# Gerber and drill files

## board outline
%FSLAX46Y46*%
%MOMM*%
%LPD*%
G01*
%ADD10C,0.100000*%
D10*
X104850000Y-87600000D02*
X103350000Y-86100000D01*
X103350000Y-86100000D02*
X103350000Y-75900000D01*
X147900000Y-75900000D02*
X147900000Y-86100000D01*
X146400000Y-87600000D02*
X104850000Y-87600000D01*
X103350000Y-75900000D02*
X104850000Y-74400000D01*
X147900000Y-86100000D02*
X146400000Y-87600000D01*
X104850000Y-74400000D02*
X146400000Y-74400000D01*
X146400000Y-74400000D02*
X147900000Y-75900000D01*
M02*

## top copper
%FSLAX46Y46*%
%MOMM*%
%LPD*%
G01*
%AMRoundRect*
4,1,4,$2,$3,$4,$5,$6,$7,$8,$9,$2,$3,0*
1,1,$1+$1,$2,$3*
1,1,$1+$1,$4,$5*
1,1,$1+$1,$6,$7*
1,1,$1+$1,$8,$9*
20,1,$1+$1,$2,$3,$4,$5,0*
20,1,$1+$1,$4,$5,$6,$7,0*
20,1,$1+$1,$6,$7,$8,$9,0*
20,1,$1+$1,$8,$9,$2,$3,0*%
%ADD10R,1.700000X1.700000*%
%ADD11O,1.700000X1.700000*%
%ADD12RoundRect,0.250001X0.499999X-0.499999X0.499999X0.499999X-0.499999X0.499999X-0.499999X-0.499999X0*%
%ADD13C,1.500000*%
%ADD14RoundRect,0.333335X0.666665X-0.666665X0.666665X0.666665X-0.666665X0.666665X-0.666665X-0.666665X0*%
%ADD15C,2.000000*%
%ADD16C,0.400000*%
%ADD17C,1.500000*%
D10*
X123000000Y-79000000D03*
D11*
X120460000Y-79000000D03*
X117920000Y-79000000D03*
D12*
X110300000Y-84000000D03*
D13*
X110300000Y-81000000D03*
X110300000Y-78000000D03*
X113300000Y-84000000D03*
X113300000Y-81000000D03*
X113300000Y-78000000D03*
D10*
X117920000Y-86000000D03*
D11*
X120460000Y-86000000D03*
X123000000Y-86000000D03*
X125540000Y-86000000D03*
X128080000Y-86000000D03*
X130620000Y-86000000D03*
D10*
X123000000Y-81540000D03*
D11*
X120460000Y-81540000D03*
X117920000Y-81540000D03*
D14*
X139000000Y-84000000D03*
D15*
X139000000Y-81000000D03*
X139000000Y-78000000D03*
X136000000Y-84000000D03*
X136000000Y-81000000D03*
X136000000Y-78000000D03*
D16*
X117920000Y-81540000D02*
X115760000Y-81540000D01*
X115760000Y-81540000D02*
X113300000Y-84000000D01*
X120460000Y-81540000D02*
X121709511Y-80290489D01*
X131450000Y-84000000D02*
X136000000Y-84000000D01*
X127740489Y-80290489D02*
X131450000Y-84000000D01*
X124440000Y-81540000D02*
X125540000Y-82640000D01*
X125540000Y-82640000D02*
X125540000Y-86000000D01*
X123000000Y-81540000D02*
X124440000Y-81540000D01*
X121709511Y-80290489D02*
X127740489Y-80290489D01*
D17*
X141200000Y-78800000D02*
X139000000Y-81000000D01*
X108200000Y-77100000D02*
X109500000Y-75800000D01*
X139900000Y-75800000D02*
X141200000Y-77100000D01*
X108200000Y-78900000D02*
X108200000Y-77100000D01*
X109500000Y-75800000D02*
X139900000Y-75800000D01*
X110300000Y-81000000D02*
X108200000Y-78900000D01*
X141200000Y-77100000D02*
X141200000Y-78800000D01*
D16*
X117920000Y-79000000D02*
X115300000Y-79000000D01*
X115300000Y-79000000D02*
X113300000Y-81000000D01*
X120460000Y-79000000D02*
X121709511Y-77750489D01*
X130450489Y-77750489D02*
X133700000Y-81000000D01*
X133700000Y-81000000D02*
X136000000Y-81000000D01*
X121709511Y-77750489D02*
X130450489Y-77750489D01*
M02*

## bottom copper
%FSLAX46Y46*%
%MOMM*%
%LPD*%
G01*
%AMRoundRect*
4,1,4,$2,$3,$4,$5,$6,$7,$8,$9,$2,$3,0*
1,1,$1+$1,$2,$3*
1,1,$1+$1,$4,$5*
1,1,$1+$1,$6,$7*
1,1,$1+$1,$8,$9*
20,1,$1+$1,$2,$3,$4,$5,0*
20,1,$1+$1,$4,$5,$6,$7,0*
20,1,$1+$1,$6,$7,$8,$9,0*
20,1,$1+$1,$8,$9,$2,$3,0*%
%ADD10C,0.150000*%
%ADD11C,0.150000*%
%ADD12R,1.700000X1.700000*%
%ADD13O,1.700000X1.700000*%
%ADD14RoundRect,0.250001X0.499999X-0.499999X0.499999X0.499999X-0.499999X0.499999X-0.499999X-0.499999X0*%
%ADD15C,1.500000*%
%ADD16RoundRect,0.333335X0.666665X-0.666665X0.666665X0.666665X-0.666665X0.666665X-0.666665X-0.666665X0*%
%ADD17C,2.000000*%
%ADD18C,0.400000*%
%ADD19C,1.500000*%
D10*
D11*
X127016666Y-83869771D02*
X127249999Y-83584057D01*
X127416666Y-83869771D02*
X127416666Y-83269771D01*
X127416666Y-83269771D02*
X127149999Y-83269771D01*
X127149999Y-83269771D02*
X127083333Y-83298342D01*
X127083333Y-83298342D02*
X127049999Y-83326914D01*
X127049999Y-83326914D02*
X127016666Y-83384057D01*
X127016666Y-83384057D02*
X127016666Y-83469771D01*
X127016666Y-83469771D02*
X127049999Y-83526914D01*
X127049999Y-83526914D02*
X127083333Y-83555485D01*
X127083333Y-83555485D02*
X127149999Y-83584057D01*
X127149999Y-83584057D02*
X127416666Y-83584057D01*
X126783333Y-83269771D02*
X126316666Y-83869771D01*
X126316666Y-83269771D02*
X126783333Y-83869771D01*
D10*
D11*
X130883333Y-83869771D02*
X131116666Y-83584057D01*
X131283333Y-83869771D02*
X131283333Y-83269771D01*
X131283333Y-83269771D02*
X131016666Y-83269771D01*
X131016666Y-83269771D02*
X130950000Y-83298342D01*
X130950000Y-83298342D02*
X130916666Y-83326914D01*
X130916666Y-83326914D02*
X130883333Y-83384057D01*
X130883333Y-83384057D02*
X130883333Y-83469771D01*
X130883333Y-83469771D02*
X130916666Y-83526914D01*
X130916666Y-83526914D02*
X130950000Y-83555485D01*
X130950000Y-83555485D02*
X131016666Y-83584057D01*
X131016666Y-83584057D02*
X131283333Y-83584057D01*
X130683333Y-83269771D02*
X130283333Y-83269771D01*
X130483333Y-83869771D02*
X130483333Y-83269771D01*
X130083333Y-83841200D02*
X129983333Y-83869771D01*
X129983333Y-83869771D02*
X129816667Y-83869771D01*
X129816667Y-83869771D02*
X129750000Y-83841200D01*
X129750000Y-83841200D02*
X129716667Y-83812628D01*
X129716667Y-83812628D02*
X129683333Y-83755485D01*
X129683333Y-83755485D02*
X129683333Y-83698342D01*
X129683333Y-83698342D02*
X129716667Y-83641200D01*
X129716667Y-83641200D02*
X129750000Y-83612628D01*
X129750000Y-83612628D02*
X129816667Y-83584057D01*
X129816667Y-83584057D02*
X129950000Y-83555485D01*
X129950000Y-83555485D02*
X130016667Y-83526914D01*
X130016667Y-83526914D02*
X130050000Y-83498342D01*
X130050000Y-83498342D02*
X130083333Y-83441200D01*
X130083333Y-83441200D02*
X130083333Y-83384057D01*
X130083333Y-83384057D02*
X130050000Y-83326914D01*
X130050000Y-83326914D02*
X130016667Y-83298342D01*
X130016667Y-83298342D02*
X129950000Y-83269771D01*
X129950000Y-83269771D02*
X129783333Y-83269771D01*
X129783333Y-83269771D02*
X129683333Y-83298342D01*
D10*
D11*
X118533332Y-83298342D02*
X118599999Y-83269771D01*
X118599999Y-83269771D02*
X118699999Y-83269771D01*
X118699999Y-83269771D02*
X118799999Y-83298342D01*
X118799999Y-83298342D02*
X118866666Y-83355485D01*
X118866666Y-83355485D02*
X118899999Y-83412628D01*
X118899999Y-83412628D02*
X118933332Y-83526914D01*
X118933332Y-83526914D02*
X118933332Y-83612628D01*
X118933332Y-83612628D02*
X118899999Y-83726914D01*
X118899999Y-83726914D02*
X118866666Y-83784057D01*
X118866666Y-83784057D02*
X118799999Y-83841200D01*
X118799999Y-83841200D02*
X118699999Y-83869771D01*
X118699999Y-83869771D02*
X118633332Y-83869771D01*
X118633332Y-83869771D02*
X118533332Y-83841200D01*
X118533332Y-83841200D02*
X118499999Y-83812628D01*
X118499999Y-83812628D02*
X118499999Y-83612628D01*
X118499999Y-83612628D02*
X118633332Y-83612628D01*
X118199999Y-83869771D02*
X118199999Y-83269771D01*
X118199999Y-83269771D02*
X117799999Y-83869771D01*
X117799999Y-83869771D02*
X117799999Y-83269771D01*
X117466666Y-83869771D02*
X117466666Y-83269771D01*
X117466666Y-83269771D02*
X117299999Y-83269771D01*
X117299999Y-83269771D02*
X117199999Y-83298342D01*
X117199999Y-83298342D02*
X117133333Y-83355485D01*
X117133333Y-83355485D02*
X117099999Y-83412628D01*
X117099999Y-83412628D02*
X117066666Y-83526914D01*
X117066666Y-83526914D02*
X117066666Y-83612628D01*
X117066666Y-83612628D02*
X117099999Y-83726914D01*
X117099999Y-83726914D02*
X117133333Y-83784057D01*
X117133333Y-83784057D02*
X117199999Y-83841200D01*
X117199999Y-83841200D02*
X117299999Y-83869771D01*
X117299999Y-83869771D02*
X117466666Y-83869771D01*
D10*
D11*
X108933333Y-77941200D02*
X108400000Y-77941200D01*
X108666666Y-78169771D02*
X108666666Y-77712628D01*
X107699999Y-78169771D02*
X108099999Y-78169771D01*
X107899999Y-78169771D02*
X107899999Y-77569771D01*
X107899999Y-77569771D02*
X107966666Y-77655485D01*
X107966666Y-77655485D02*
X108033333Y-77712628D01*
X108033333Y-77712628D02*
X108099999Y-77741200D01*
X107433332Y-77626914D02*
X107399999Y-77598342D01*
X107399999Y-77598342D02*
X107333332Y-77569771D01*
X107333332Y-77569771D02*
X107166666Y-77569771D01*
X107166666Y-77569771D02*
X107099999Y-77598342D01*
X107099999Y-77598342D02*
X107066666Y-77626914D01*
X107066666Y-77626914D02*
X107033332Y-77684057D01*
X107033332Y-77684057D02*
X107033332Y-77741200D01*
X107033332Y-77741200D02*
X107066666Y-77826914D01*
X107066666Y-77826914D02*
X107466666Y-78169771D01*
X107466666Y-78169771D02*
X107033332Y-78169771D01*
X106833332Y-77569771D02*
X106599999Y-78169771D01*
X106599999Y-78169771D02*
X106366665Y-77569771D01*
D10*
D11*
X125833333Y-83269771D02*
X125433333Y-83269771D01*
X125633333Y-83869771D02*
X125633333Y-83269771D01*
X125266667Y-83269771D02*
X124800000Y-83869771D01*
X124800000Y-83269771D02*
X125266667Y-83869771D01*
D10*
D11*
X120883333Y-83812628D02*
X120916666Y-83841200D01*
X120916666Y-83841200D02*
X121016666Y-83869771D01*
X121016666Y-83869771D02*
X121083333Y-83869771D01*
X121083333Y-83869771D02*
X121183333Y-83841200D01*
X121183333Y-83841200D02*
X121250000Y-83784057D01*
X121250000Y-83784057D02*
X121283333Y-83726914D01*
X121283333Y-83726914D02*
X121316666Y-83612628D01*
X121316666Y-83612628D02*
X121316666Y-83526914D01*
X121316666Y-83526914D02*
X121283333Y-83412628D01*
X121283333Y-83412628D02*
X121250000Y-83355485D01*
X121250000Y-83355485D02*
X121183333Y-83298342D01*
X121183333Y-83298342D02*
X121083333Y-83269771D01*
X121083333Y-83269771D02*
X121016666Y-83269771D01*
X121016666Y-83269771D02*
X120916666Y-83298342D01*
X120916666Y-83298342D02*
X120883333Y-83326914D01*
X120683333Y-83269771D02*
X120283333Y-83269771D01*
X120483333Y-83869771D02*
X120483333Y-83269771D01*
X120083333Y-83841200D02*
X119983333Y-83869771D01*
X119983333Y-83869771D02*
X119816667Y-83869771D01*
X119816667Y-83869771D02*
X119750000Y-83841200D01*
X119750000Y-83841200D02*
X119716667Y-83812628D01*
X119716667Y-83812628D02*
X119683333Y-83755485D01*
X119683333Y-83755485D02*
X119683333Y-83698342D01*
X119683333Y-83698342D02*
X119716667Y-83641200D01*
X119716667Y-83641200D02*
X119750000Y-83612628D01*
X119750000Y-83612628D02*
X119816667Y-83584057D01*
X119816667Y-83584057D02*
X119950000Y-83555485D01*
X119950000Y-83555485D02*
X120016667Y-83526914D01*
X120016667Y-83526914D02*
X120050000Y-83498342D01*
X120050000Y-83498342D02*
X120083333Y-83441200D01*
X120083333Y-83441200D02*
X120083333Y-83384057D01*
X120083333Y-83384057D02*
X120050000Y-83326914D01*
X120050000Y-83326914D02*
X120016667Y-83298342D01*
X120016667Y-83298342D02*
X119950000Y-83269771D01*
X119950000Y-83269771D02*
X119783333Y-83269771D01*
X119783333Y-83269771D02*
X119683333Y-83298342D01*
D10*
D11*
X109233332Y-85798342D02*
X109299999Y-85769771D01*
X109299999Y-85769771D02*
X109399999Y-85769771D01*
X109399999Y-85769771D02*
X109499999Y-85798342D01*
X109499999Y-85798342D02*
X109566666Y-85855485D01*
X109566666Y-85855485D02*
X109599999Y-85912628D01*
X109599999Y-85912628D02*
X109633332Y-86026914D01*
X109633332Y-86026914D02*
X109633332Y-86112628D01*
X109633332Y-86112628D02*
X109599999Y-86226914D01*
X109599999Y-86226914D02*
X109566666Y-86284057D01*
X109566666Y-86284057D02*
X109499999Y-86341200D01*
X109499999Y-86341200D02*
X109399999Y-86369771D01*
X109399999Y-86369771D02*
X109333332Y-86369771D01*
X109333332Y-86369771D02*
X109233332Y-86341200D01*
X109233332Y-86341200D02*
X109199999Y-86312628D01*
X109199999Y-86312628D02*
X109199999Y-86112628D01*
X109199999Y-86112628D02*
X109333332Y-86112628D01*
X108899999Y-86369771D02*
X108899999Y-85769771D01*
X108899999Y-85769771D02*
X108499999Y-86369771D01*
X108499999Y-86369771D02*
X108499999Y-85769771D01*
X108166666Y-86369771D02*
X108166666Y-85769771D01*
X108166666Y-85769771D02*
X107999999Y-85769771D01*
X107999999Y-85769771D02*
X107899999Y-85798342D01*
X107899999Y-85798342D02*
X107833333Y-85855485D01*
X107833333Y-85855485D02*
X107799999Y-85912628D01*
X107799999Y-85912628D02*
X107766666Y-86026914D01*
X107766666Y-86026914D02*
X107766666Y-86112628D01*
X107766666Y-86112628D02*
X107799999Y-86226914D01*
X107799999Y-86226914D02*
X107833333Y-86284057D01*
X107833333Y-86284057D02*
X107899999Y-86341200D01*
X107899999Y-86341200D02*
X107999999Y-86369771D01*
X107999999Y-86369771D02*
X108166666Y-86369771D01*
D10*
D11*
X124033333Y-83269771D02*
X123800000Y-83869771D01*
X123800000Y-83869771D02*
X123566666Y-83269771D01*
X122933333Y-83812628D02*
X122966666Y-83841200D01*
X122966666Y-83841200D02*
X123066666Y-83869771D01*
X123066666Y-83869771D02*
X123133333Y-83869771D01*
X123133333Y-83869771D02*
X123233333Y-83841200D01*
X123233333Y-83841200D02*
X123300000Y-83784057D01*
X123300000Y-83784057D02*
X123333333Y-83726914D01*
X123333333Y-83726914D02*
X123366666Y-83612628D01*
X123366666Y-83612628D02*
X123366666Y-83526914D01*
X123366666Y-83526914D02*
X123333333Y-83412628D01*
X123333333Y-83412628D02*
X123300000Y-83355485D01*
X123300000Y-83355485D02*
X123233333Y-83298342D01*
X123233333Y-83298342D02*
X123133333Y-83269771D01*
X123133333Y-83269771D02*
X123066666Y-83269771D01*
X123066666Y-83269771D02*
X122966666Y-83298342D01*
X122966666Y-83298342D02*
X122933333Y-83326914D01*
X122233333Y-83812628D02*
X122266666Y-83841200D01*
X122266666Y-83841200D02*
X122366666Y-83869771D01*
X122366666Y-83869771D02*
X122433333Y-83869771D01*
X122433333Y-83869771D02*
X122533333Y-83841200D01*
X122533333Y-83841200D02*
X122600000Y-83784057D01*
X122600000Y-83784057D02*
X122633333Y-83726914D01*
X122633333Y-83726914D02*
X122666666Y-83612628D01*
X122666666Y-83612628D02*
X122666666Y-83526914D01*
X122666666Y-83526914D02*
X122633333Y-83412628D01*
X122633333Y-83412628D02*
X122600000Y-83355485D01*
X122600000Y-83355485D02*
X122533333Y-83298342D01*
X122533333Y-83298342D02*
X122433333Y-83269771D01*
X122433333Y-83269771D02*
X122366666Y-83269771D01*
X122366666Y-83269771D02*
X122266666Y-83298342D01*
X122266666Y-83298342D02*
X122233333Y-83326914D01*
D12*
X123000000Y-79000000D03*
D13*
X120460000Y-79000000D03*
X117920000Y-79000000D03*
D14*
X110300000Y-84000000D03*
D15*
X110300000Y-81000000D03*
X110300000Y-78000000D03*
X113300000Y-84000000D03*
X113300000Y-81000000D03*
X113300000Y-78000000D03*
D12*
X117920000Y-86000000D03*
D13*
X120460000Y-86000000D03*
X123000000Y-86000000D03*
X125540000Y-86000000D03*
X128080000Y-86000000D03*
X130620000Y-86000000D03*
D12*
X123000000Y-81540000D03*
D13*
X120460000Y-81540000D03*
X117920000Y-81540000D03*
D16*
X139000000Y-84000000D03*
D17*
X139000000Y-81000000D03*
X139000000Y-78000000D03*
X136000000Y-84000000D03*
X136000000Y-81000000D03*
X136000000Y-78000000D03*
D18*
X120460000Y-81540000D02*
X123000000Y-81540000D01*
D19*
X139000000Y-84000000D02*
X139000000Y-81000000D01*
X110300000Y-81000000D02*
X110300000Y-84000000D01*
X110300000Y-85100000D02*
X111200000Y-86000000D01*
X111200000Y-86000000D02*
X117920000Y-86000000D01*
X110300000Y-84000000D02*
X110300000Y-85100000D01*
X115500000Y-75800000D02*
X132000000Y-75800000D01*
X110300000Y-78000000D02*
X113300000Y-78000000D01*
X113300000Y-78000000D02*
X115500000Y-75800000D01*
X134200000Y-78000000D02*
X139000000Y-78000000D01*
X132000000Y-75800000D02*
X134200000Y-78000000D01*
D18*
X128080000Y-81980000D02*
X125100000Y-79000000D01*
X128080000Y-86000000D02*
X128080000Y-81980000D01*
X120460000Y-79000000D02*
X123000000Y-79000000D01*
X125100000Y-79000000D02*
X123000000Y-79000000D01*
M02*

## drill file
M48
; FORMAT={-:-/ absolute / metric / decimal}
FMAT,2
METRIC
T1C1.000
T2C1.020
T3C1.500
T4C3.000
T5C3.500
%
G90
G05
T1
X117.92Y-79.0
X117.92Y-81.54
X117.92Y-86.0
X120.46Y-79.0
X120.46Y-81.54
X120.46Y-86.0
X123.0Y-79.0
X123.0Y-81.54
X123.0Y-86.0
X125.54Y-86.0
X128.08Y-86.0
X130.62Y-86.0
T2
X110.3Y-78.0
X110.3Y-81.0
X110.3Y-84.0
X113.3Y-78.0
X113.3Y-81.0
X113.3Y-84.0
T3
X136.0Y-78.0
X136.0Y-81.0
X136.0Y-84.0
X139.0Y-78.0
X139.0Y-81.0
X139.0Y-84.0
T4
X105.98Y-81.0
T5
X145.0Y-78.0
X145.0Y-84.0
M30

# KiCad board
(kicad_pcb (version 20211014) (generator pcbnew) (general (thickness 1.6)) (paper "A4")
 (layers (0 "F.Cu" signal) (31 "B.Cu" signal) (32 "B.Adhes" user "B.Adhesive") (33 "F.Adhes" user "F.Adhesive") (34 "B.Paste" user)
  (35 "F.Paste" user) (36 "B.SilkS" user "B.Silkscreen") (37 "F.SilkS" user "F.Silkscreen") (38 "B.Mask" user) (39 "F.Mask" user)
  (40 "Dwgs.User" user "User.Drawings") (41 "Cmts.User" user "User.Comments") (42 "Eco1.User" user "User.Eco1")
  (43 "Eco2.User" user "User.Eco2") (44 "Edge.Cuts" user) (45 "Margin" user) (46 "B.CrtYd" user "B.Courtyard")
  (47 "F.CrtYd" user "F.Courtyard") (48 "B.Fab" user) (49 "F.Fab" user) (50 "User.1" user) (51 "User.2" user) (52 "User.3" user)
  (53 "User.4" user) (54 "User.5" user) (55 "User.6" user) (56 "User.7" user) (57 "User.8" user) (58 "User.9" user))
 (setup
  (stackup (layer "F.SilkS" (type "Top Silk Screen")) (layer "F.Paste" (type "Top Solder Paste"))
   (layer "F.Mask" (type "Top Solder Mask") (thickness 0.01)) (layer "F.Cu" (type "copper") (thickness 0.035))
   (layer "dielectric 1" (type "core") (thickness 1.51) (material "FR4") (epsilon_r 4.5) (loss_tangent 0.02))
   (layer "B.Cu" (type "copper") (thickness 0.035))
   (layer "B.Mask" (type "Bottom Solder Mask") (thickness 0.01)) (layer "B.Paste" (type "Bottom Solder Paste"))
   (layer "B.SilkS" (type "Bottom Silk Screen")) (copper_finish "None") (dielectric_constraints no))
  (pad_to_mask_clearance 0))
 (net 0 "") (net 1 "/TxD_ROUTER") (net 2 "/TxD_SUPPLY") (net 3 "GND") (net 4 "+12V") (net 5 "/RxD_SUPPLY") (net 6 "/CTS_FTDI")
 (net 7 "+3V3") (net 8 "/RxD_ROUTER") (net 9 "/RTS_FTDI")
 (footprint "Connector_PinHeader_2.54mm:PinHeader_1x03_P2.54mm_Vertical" (layer "F.Cu") (at 123 79 -90)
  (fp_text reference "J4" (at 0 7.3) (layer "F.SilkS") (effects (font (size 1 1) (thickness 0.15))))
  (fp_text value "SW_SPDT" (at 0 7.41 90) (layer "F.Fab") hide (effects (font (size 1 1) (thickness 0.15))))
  (pad "1" thru_hole rect (at 0 0 270) (size 1.7 1.7) (drill 1) (layers *.Cu *.Mask) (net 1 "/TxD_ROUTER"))
  (pad "2" thru_hole oval (at 0 2.54 270) (size 1.7 1.7) (drill 1) (layers *.Cu *.Mask) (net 1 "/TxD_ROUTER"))
  (pad "3" thru_hole oval (at 0 5.08 270) (size 1.7 1.7) (drill 1) (layers *.Cu *.Mask) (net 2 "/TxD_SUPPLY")))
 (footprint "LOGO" (layer "F.Cu") (at 128 78.8)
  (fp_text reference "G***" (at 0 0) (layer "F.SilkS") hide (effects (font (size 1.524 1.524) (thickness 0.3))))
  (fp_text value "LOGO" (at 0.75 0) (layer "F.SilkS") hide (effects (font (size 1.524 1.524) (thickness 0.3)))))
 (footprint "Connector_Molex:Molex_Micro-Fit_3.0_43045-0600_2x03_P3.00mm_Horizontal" (layer "F.Cu") (at 110.3 84 90)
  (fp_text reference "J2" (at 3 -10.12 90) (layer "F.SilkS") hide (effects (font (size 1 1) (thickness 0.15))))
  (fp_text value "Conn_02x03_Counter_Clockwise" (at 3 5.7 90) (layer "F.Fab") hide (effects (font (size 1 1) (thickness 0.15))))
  (pad "" np_thru_hole circle (at 3 -4.32 90) (size 3 3) (drill 3) (layers *.Cu *.Mask))
  (pad "1" thru_hole roundrect (at 0 0 90) (size 1.5 1.5) (drill 1.02) (layers *.Cu *.Mask) (roundrect_rratio 0.1666673333) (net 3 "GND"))
  (pad "2" thru_hole circle (at 3 0 90) (size 1.5 1.5) (drill 1.02) (layers *.Cu *.Mask) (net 3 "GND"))
  (pad "3" thru_hole circle (at 6 0 90) (size 1.5 1.5) (drill 1.02) (layers *.Cu *.Mask) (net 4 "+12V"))
  (pad "4" thru_hole circle (at 0 3 90) (size 1.5 1.5) (drill 1.02) (layers *.Cu *.Mask) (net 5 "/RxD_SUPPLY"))
  (pad "5" thru_hole circle (at 3 3 90) (size 1.5 1.5) (drill 1.02) (layers *.Cu *.Mask) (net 2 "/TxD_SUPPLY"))
  (pad "6" thru_hole circle (at 6 3 90) (size 1.5 1.5) (drill 1.02) (layers *.Cu *.Mask) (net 4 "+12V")))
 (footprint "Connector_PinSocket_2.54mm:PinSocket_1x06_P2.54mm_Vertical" (layer "F.Cu") (at 117.92 86 90)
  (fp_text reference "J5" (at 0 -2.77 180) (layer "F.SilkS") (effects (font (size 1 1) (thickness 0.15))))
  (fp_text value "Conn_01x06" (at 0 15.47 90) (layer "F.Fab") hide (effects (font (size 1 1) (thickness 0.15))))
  (pad "1" thru_hole rect (at 0 0 90) (size 1.7 1.7) (drill 1) (layers *.Cu *.Mask) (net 3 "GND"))
  (pad "2" thru_hole oval (at 0 2.54 90) (size 1.7 1.7) (drill 1) (layers *.Cu *.Mask) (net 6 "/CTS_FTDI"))
  (pad "3" thru_hole oval (at 0 5.08 90) (size 1.7 1.7) (drill 1) (layers *.Cu *.Mask) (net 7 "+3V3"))
  (pad "4" thru_hole oval (at 0 7.62 90) (size 1.7 1.7) (drill 1) (layers *.Cu *.Mask) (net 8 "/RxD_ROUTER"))
  (pad "5" thru_hole oval (at 0 10.16 90) (size 1.7 1.7) (drill 1) (layers *.Cu *.Mask) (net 1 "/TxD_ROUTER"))
  (pad "6" thru_hole oval (at 0 12.7 90) (size 1.7 1.7) (drill 1) (layers *.Cu *.Mask) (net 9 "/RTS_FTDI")))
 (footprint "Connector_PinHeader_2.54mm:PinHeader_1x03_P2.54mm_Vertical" (layer "F.Cu") (at 123 81.54 -90)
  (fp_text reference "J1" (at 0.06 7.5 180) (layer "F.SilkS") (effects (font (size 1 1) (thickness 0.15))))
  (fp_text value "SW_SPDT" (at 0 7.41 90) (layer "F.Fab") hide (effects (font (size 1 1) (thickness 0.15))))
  (pad "1" thru_hole rect (at 0 0 270) (size 1.7 1.7) (drill 1) (layers *.Cu *.Mask) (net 8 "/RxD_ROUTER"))
  (pad "2" thru_hole oval (at 0 2.54 270) (size 1.7 1.7) (drill 1) (layers *.Cu *.Mask) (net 8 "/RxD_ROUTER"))
  (pad "3" thru_hole oval (at 0 5.08 270) (size 1.7 1.7) (drill 1) (layers *.Cu *.Mask) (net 5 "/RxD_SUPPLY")))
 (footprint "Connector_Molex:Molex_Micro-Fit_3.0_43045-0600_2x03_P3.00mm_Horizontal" (layer "B.Cu") (at 139 84 90)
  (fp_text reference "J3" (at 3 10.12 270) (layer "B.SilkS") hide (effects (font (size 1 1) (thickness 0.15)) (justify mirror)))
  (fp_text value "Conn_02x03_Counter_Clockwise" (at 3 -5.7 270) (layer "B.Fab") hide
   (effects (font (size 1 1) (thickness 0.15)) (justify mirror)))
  (pad "" np_thru_hole circle (at 6 6 90) (size 3.5 3.5) (drill 3.5) (layers F&B.Cu *.Mask))
  (pad "" np_thru_hole circle (at 0 6 90) (size 3.5 3.5) (drill 3.5) (layers F&B.Cu *.Mask))
  (pad "1" thru_hole roundrect (at 0 0 90) (size 2 2) (drill 1.5) (layers *.Cu *.Mask) (roundrect_rratio 0.1666675) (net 3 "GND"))
  (pad "2" thru_hole circle (at 3 0 90) (size 2 2) (drill 1.5) (layers *.Cu *.Mask) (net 3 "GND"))
  (pad "3" thru_hole circle (at 6 0 90) (size 2 2) (drill 1.5) (layers *.Cu *.Mask) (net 4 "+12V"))
  (pad "4" thru_hole circle (at 0 -3 90) (size 2 2) (drill 1.5) (layers *.Cu *.Mask) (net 8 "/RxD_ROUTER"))
  (pad "5" thru_hole circle (at 3 -3 90) (size 2 2) (drill 1.5) (layers *.Cu *.Mask) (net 1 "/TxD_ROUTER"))
  (pad "6" thru_hole circle (at 6 -3 90) (size 2 2) (drill 1.5) (layers *.Cu *.Mask) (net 4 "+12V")))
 (gr_line (start 104.85 87.6) (end 103.35 86.1) (layer "Edge.Cuts") (width 0.1))
 (gr_line (start 103.35 86.1) (end 103.35 75.9) (layer "Edge.Cuts") (width 0.1))
 (gr_line locked (start 147.9 75.9) (end 147.9 86.1) (layer "Edge.Cuts") (width 0.1))
 (gr_line (start 146.4 87.6) (end 104.85 87.6) (layer "Edge.Cuts") (width 0.1))
 (gr_line (start 103.35 75.9) (end 104.85 74.4) (layer "Edge.Cuts") (width 0.1))
 (gr_line (start 147.9 86.1) (end 146.4 87.6) (layer "Edge.Cuts") (width 0.1))
 (gr_line (start 104.85 74.4) (end 146.4 74.4) (layer "Edge.Cuts") (width 0.1))
 (gr_line (start 146.4 74.4) (end 147.9 75.9) (layer "Edge.Cuts") (width 0.1))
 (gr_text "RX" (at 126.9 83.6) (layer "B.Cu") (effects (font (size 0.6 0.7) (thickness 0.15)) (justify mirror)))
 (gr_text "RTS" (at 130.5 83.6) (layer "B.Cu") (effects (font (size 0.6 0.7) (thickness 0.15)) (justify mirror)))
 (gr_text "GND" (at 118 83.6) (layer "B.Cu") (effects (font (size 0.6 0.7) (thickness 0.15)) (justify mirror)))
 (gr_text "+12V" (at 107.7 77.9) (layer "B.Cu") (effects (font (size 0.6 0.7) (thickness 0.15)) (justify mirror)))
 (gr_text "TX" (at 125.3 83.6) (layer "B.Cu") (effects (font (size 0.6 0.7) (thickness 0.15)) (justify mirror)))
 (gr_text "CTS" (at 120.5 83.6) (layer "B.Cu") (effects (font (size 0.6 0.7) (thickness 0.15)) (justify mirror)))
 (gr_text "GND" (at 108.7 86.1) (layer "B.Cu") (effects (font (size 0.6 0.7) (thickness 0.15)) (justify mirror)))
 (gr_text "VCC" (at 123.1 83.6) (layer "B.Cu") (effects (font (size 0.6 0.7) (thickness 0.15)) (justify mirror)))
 (segment (start 117.92 81.54) (end 115.76 81.54) (width 0.4) (layer "F.Cu") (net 5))
 (segment (start 115.76 81.54) (end 113.3 84) (width 0.4) (layer "F.Cu") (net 5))
 (segment (start 120.46 81.54) (end 121.709511 80.290489) (width 0.4) (layer "F.Cu") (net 8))
 (segment (start 131.45 84) (end 136 84) (width 0.4) (layer "F.Cu") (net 8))
 (segment (start 127.740489 80.290489) (end 131.45 84) (width 0.4) (layer "F.Cu") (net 8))
 (segment (start 124.44 81.54) (end 125.54 82.64) (width 0.4) (layer "F.Cu") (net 8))
 (segment (start 125.54 82.64) (end 125.54 86) (width 0.4) (layer "F.Cu") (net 8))
 (segment (start 123 81.54) (end 124.44 81.54) (width 0.4) (layer "F.Cu") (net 8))
 (segment (start 121.709511 80.290489) (end 127.740489 80.290489) (width 0.4) (layer "F.Cu") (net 8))
 (segment (start 120.46 81.54) (end 123 81.54) (width 0.4) (layer "B.Cu") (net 8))
 (segment (start 141.2 78.8) (end 139 81) (width 1.5) (layer "F.Cu") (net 3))
 (segment (start 108.2 77.1) (end 109.5 75.8) (width 1.5) (layer "F.Cu") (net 3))
 (segment (start 139.9 75.8) (end 141.2 77.1) (width 1.5) (layer "F.Cu") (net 3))
 (segment (start 108.2 78.9) (end 108.2 77.1) (width 1.5) (layer "F.Cu") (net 3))
 (segment (start 109.5 75.8) (end 139.9 75.8) (width 1.5) (layer "F.Cu") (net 3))
 (segment (start 110.3 81) (end 108.2 78.9) (width 1.5) (layer "F.Cu") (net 3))
 (segment (start 141.2 77.1) (end 141.2 78.8) (width 1.5) (layer "F.Cu") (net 3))
 (segment (start 139 84) (end 139 81) (width 1.5) (layer "B.Cu") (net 3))
 (segment (start 110.3 81) (end 110.3 84) (width 1.5) (layer "B.Cu") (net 3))
 (segment (start 110.3 85.1) (end 111.2 86) (width 1.5) (layer "B.Cu") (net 3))
 (segment (start 111.2 86) (end 117.92 86) (width 1.5) (layer "B.Cu") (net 3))
 (segment (start 110.3 84) (end 110.3 85.1) (width 1.5) (layer "B.Cu") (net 3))
 (segment (start 115.5 75.8) (end 132 75.8) (width 1.5) (layer "B.Cu") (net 4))
 (segment (start 110.3 78) (end 113.3 78) (width 1.5) (layer "B.Cu") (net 4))
 (segment (start 113.3 78) (end 115.5 75.8) (width 1.5) (layer "B.Cu") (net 4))
 (segment (start 134.2 78) (end 139 78) (width 1.5) (layer "B.Cu") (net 4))
 (segment (start 132 75.8) (end 134.2 78) (width 1.5) (layer "B.Cu") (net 4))
 (segment (start 117.92 79) (end 115.3 79) (width 0.4) (layer "F.Cu") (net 2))
 (segment (start 115.3 79) (end 113.3 81) (width 0.4) (layer "F.Cu") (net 2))
 (segment (start 120.46 79) (end 121.709511 77.750489) (width 0.4) (layer "F.Cu") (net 1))
 (segment (start 130.450489 77.750489) (end 133.7 81) (width 0.4) (layer "F.Cu") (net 1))
 (segment (start 133.7 81) (end 136 81) (width 0.4) (layer "F.Cu") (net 1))
 (segment (start 121.709511 77.750489) (end 130.450489 77.750489) (width 0.4) (layer "F.Cu") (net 1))
 (segment (start 128.08 81.98) (end 125.1 79) (width 0.4) (layer "B.Cu") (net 1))
 (segment (start 128.08 86) (end 128.08 81.98) (width 0.4) (layer "B.Cu") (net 1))
 (segment (start 120.46 79) (end 123 79) (width 0.4) (layer "B.Cu") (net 1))
 (segment (start 125.1 79) (end 123 79) (width 0.4) (layer "B.Cu") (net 1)))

